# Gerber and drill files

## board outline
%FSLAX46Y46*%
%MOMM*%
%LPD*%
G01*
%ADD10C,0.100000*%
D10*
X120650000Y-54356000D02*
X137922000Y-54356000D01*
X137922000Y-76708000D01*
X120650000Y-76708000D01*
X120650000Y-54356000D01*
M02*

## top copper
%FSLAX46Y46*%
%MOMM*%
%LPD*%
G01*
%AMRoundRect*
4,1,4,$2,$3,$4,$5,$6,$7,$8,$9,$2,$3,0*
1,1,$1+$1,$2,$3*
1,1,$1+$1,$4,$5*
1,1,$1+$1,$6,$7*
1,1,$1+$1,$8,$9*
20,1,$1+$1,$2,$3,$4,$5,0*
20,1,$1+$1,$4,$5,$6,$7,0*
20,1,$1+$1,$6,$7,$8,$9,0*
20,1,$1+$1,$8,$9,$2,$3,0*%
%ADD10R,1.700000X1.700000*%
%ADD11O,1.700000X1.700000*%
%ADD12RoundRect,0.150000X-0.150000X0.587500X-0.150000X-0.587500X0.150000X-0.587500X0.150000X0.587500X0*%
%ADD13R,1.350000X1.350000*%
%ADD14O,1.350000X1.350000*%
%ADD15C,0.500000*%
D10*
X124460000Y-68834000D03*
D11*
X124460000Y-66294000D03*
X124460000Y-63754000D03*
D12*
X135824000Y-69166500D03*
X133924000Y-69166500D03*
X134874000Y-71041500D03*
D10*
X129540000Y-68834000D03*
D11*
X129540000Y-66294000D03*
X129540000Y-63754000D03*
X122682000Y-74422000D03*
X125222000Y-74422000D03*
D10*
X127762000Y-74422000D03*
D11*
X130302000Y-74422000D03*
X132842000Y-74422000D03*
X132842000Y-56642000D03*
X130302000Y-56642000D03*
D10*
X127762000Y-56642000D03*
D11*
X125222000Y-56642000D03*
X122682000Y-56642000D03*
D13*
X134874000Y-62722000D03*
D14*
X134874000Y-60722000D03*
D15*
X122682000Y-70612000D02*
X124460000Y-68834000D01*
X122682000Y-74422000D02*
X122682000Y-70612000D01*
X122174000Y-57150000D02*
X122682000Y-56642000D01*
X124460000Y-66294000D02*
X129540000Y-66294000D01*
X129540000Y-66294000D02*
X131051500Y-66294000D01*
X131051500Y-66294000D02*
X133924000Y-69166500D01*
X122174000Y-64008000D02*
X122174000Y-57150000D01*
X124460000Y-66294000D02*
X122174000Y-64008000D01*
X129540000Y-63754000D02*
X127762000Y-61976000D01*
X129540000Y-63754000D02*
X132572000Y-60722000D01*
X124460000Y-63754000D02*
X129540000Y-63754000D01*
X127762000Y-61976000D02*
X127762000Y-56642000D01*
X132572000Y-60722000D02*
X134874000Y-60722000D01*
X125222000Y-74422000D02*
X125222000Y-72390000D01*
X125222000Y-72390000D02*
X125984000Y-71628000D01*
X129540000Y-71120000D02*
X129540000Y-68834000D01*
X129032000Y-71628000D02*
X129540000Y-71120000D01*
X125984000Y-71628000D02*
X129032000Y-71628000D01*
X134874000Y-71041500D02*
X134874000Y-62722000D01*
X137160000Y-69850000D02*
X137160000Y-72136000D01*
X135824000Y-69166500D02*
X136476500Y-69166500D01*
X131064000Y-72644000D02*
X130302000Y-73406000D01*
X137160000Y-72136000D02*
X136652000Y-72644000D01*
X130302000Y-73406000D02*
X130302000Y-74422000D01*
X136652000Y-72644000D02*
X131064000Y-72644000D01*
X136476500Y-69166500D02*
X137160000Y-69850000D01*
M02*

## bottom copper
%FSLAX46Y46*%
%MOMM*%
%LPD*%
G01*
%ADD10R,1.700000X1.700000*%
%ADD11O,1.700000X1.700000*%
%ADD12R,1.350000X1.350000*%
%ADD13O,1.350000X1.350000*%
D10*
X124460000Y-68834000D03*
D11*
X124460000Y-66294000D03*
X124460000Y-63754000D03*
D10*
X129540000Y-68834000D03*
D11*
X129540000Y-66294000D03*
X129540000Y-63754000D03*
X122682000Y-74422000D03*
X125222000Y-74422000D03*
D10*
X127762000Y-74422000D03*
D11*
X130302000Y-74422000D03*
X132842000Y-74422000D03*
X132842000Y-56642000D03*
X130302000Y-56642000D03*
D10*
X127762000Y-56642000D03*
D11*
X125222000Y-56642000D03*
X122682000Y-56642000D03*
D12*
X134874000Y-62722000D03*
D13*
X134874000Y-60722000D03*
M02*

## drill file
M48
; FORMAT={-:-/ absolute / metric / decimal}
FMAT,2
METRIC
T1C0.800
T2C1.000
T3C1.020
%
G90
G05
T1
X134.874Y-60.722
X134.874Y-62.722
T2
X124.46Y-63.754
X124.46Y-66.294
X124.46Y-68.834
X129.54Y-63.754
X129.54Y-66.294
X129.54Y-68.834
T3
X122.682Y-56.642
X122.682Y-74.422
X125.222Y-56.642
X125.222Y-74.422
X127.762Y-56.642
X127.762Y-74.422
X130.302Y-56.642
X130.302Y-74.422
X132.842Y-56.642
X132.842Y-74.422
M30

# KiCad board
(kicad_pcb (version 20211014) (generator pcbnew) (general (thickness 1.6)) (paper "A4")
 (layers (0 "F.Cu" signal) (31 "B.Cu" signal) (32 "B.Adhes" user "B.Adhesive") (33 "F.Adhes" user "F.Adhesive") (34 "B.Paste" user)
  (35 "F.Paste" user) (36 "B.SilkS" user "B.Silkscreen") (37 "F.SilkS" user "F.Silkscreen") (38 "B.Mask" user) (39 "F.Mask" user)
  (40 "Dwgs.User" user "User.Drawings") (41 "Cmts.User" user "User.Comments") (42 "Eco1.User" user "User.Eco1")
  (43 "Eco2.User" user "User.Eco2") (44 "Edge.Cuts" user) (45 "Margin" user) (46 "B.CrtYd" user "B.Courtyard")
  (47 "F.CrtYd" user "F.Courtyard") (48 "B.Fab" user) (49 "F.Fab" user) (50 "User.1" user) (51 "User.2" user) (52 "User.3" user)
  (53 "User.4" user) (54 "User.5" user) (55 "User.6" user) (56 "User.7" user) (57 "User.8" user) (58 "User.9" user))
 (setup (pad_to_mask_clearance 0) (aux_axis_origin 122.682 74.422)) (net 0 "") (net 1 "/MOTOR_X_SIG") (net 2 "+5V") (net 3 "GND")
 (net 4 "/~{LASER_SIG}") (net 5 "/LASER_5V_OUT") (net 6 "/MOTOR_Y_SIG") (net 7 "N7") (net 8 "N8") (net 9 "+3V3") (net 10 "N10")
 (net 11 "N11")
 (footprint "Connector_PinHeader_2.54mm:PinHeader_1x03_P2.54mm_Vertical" (layer "F.Cu") (at 124.46 68.834 180)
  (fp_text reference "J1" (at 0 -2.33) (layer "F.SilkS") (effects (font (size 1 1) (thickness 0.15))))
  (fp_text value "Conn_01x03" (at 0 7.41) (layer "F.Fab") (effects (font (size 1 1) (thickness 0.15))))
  (pad "1" thru_hole rect (at 0 0 180) (size 1.7 1.7) (drill 1) (layers *.Cu *.Mask) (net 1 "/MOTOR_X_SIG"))
  (pad "2" thru_hole oval (at 0 2.54 180) (size 1.7 1.7) (drill 1) (layers *.Cu *.Mask) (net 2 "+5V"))
  (pad "3" thru_hole oval (at 0 5.08 180) (size 1.7 1.7) (drill 1) (layers *.Cu *.Mask) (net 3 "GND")))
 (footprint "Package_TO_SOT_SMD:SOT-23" (layer "F.Cu") (at 134.874 70.104 -90)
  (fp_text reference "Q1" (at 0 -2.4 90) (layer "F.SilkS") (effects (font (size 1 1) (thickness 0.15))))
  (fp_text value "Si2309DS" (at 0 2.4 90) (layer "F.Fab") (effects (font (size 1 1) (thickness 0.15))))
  (pad "1" smd roundrect (at -0.9375 -0.95 270) (size 1.475 0.6) (layers "F.Cu" "F.Paste" "F.Mask") (roundrect_rratio 0.25)
   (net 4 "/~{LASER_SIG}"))
  (pad "2" smd roundrect (at -0.9375 0.95 270) (size 1.475 0.6) (layers "F.Cu" "F.Paste" "F.Mask") (roundrect_rratio 0.25) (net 2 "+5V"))
  (pad "3" smd roundrect (at 0.9375 0 270) (size 1.475 0.6) (layers "F.Cu" "F.Paste" "F.Mask") (roundrect_rratio 0.25)
   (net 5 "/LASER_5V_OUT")))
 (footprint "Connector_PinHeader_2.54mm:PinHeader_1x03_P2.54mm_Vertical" (layer "F.Cu") (at 129.54 68.834 180)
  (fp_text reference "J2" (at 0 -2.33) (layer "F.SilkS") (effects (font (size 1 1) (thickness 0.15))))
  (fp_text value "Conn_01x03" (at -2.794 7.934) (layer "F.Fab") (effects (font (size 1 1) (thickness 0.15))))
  (pad "1" thru_hole rect (at 0 0 180) (size 1.7 1.7) (drill 1) (layers *.Cu *.Mask) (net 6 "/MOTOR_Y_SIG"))
  (pad "2" thru_hole oval (at 0 2.54 180) (size 1.7 1.7) (drill 1) (layers *.Cu *.Mask) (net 2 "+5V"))
  (pad "3" thru_hole oval (at 0 5.08 180) (size 1.7 1.7) (drill 1) (layers *.Cu *.Mask) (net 3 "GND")))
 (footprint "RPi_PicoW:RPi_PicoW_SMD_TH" (layer "F.Cu") (at 146.812 65.532 90)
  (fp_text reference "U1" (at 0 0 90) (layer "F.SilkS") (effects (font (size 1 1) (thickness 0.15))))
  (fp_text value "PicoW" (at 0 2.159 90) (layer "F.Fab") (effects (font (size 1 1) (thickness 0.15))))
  (pad "1" thru_hole oval (at -8.89 -24.13 90) (size 1.7 1.7) (drill 1.02) (layers *.Cu *.Mask) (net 1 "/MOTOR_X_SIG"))
  (pad "2" thru_hole oval (at -8.89 -21.59 90) (size 1.7 1.7) (drill 1.02) (layers *.Cu *.Mask) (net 6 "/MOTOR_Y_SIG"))
  (pad "3" thru_hole rect (at -8.89 -19.05 90) (size 1.7 1.7) (drill 1.02) (layers *.Cu *.Mask) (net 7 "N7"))
  (pad "4" thru_hole oval (at -8.89 -16.51 90) (size 1.7 1.7) (drill 1.02) (layers *.Cu *.Mask) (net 4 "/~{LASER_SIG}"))
  (pad "5" thru_hole oval (at -8.89 -13.97 90) (size 1.7 1.7) (drill 1.02) (layers *.Cu *.Mask) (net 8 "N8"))
  (pad "36" thru_hole oval (at 8.89 -13.97 90) (size 1.7 1.7) (drill 1.02) (layers *.Cu *.Mask) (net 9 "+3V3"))
  (pad "37" thru_hole oval (at 8.89 -16.51 90) (size 1.7 1.7) (drill 1.02) (layers *.Cu *.Mask) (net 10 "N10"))
  (pad "38" thru_hole rect (at 8.89 -19.05 90) (size 1.7 1.7) (drill 1.02) (layers *.Cu *.Mask) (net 3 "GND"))
  (pad "39" thru_hole oval (at 8.89 -21.59 90) (size 1.7 1.7) (drill 1.02) (layers *.Cu *.Mask) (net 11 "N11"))
  (pad "40" thru_hole oval (at 8.89 -24.13 90) (size 1.7 1.7) (drill 1.02) (layers *.Cu *.Mask) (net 2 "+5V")))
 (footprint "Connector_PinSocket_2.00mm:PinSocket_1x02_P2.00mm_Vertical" (layer "F.Cu") (at 134.874 62.722 180)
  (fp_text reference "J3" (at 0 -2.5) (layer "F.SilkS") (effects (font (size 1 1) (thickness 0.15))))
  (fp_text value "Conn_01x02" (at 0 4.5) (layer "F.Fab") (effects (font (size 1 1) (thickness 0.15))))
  (pad "1" thru_hole rect (at 0 0 180) (size 1.35 1.35) (drill 0.8) (layers *.Cu *.Mask) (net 5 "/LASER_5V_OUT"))
  (pad "2" thru_hole oval (at 0 2 180) (size 1.35 1.35) (drill 0.8) (layers *.Cu *.Mask) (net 3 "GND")))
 (gr_rect (start 120.65 54.356) (end 137.922 76.708) (layer "Edge.Cuts") (width 0.1) (fill none))
 (segment (start 122.682 70.612) (end 124.46 68.834) (width 0.5) (layer "F.Cu") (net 1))
 (segment (start 122.682 74.422) (end 122.682 70.612) (width 0.5) (layer "F.Cu") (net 1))
 (segment (start 122.174 57.15) (end 122.682 56.642) (width 0.5) (layer "F.Cu") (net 2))
 (segment (start 124.46 66.294) (end 129.54 66.294) (width 0.5) (layer "F.Cu") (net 2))
 (segment (start 129.54 66.294) (end 131.0515 66.294) (width 0.5) (layer "F.Cu") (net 2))
 (segment (start 131.0515 66.294) (end 133.924 69.1665) (width 0.5) (layer "F.Cu") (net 2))
 (segment (start 122.174 64.008) (end 122.174 57.15) (width 0.5) (layer "F.Cu") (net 2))
 (segment (start 124.46 66.294) (end 122.174 64.008) (width 0.5) (layer "F.Cu") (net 2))
 (segment (start 129.54 63.754) (end 127.762 61.976) (width 0.5) (layer "F.Cu") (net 3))
 (segment (start 129.54 63.754) (end 132.572 60.722) (width 0.5) (layer "F.Cu") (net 3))
 (segment (start 124.46 63.754) (end 129.54 63.754) (width 0.5) (layer "F.Cu") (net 3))
 (segment (start 127.762 61.976) (end 127.762 56.642) (width 0.5) (layer "F.Cu") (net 3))
 (segment (start 132.572 60.722) (end 134.874 60.722) (width 0.5) (layer "F.Cu") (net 3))
 (segment (start 125.222 74.422) (end 125.222 72.39) (width 0.5) (layer "F.Cu") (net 6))
 (segment (start 125.222 72.39) (end 125.984 71.628) (width 0.5) (layer "F.Cu") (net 6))
 (segment (start 129.54 71.12) (end 129.54 68.834) (width 0.5) (layer "F.Cu") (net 6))
 (segment (start 129.032 71.628) (end 129.54 71.12) (width 0.5) (layer "F.Cu") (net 6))
 (segment (start 125.984 71.628) (end 129.032 71.628) (width 0.5) (layer "F.Cu") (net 6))
 (segment (start 134.874 71.0415) (end 134.874 62.722) (width 0.5) (layer "F.Cu") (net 5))
 (segment (start 137.16 69.85) (end 137.16 72.136) (width 0.5) (layer "F.Cu") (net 4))
 (segment (start 135.824 69.1665) (end 136.4765 69.1665) (width 0.5) (layer "F.Cu") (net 4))
 (segment (start 131.064 72.644) (end 130.302 73.406) (width 0.5) (layer "F.Cu") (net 4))
 (segment (start 137.16 72.136) (end 136.652 72.644) (width 0.5) (layer "F.Cu") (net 4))
 (segment (start 130.302 73.406) (end 130.302 74.422) (width 0.5) (layer "F.Cu") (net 4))
 (segment (start 136.652 72.644) (end 131.064 72.644) (width 0.5) (layer "F.Cu") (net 4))
 (segment (start 136.4765 69.1665) (end 137.16 69.85) (width 0.5) (layer "F.Cu") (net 4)))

